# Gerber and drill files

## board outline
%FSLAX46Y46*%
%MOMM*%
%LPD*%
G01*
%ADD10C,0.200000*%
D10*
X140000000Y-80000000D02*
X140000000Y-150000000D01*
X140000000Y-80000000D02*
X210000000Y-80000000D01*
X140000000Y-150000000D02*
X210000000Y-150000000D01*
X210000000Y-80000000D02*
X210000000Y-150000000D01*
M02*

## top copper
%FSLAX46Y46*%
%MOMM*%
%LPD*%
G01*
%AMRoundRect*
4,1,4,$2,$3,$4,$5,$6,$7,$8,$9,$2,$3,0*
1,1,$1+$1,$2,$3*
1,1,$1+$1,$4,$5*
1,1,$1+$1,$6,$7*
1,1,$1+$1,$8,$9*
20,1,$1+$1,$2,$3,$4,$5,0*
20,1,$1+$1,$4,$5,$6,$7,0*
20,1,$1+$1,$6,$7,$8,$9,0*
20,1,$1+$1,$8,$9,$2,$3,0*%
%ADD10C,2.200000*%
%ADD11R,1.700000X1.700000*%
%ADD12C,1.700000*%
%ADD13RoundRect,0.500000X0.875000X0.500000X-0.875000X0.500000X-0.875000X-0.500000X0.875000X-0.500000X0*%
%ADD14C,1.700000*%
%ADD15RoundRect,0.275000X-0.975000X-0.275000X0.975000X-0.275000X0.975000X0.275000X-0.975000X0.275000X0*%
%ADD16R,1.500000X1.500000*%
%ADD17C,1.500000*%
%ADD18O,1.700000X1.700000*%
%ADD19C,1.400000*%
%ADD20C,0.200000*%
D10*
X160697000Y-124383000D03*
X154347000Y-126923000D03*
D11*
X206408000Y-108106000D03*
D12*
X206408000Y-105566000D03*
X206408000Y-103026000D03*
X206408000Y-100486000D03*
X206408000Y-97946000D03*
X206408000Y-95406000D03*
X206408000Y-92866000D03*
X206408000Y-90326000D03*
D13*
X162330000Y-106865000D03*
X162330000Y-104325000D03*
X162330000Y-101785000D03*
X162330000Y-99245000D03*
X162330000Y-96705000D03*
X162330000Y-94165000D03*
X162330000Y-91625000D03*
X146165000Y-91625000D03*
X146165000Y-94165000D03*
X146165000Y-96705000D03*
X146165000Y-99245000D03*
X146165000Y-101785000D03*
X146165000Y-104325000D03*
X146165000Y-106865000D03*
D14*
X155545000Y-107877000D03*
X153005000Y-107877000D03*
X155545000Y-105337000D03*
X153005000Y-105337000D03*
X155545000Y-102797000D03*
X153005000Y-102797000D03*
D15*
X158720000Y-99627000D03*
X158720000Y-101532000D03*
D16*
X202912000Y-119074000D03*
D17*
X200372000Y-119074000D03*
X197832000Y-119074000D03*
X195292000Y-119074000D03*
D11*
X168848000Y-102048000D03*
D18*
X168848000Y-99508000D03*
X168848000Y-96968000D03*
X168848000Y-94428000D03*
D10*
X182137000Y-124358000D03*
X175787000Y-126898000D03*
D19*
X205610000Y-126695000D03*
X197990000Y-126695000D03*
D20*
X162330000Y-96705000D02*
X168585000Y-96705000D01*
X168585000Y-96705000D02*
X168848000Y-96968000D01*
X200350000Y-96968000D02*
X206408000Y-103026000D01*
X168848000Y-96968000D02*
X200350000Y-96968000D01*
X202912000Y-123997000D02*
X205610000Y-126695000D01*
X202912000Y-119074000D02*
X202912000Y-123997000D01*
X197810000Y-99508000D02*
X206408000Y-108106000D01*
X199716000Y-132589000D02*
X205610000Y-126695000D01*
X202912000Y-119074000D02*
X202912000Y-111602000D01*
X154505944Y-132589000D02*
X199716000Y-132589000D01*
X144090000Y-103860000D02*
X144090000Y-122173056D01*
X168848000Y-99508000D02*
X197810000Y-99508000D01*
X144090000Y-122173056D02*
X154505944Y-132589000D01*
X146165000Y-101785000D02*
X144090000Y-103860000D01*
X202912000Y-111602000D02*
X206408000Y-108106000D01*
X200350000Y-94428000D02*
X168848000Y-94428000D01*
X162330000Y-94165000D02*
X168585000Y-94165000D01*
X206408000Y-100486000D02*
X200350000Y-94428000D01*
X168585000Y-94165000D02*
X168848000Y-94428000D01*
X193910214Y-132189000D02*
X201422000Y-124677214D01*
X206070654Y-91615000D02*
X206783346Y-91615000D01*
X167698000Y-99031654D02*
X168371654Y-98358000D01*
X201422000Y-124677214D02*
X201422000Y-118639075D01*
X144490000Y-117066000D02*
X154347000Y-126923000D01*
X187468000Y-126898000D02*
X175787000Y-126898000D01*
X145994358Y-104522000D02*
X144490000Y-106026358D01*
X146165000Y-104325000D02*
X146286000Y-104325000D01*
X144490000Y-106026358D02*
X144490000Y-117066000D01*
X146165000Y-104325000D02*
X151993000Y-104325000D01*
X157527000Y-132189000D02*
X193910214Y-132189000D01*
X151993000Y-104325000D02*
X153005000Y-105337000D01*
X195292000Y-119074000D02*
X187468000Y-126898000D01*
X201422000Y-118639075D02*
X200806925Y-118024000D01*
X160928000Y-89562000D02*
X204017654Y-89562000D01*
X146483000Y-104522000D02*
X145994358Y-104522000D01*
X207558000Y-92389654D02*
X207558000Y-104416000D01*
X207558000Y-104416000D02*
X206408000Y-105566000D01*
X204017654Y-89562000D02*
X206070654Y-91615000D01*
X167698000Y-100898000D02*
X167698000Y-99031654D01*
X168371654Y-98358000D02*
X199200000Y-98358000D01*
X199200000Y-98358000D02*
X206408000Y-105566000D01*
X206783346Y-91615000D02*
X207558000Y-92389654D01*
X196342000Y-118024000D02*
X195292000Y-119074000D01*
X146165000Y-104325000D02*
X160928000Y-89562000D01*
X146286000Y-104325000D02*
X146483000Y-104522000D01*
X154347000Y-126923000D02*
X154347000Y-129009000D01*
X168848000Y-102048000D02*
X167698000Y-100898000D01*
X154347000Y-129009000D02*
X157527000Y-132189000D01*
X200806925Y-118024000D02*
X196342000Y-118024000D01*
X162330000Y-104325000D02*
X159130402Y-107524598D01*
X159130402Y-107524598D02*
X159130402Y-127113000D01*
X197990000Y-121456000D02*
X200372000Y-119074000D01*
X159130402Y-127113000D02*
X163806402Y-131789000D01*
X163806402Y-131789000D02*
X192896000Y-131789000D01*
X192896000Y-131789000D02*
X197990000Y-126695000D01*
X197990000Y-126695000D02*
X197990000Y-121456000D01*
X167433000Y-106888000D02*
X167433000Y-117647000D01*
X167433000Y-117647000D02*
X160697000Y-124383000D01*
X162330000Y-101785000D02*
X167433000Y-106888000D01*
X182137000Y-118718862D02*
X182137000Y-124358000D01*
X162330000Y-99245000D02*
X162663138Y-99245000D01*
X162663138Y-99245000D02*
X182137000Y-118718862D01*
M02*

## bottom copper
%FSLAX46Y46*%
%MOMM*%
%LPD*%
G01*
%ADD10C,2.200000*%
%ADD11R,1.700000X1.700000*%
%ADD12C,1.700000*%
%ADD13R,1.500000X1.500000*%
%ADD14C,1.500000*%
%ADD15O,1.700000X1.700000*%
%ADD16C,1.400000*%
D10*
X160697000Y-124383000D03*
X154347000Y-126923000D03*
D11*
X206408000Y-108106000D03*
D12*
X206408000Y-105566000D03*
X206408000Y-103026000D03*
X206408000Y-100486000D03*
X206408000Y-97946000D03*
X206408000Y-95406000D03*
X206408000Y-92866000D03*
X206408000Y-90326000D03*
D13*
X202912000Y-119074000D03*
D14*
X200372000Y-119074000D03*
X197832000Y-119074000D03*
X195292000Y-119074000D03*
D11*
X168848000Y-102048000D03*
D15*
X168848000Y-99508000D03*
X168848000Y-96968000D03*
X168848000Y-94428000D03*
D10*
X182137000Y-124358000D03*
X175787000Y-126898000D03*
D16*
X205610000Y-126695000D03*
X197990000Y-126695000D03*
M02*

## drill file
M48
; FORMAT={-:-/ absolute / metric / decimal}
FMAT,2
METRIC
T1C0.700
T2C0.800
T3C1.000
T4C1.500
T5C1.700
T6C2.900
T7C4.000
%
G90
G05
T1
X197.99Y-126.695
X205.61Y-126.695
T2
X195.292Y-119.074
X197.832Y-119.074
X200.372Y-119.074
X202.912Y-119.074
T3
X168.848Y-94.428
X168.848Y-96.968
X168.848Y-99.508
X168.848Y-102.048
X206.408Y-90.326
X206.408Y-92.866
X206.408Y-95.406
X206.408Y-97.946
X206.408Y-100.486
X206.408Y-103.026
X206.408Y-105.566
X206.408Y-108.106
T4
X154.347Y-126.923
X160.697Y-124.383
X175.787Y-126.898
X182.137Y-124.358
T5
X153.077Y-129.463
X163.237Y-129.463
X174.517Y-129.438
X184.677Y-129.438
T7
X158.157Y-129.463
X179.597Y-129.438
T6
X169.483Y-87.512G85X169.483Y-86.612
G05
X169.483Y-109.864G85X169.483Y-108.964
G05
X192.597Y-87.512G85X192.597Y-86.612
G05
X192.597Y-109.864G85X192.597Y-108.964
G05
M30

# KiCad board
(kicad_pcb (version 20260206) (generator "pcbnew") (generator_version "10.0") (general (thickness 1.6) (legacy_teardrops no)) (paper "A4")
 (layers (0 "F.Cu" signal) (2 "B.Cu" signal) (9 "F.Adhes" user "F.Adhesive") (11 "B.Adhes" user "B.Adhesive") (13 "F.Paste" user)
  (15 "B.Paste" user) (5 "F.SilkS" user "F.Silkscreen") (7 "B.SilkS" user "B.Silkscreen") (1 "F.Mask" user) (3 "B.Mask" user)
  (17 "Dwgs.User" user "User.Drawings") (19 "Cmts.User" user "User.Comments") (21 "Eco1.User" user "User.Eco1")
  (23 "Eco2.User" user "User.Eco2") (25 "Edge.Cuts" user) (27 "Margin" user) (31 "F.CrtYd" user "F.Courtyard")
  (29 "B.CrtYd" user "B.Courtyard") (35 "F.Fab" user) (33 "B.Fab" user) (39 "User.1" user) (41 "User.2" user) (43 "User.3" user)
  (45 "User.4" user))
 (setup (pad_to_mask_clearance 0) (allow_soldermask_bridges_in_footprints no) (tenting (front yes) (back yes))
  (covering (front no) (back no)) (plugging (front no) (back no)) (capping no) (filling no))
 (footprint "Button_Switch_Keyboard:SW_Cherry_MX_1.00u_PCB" (layer "F.Cu") (at 160.697 124.383)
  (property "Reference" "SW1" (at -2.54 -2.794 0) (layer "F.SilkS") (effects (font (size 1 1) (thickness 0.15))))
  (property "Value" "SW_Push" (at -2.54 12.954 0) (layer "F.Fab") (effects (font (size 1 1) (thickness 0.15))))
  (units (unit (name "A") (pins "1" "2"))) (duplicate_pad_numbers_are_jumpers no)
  (pad "" np_thru_hole circle (at -7.62 5.08) (size 1.7 1.7) (drill 1.7) (layers "*.Cu" "*.Mask"))
  (pad "" np_thru_hole circle (at -2.54 5.08) (size 4 4) (drill 4) (layers "*.Cu" "*.Mask"))
  (pad "" np_thru_hole circle (at 2.54 5.08) (size 1.7 1.7) (drill 1.7) (layers "*.Cu" "*.Mask"))
  (pad "1" thru_hole circle (at 0 0) (size 2.2 2.2) (drill 1.5) (layers "*.Cu" "*.Mask") (remove_unused_layers no) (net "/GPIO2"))
  (pad "2" thru_hole circle (at -6.35 2.54) (size 2.2 2.2) (drill 1.5) (layers "*.Cu" "*.Mask") (remove_unused_layers no) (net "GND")))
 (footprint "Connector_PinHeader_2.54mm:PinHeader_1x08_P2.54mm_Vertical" (layer "F.Cu") (at 206.408 108.106 180)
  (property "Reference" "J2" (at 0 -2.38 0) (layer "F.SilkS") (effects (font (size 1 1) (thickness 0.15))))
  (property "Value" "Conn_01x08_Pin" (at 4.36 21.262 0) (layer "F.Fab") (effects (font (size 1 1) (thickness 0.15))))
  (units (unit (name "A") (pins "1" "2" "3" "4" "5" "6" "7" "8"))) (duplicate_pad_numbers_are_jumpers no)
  (pad "1" thru_hole rect (at 0 0 180) (size 1.7 1.7) (drill 1) (layers "*.Cu" "*.Mask") (remove_unused_layers no) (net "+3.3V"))
  (pad "2" thru_hole circle (at 0 2.54 180) (size 1.7 1.7) (drill 1) (layers "*.Cu" "*.Mask") (remove_unused_layers no) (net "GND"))
  (pad "3" thru_hole circle (at 0 5.08 180) (size 1.7 1.7) (drill 1) (layers "*.Cu" "*.Mask") (remove_unused_layers no) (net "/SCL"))
  (pad "4" thru_hole circle (at 0 7.62 180) (size 1.7 1.7) (drill 1) (layers "*.Cu" "*.Mask") (remove_unused_layers no) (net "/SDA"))
  (pad "5" thru_hole circle (at 0 10.16 180) (size 1.7 1.7) (drill 1) (layers "*.Cu" "*.Mask") (remove_unused_layers no)
   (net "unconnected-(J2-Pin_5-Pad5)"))
  (pad "6" thru_hole circle (at 0 12.7 180) (size 1.7 1.7) (drill 1) (layers "*.Cu" "*.Mask") (remove_unused_layers no)
   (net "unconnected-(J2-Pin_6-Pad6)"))
  (pad "7" thru_hole circle (at 0 15.24 180) (size 1.7 1.7) (drill 1) (layers "*.Cu" "*.Mask") (remove_unused_layers no)
   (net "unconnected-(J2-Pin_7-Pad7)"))
  (pad "8" thru_hole circle (at 0 17.78 180) (size 1.7 1.7) (drill 1) (layers "*.Cu" "*.Mask") (remove_unused_layers no)
   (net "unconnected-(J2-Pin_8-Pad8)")))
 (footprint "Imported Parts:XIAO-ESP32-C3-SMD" (layer "F.Cu") (at 163.165 88.745 180)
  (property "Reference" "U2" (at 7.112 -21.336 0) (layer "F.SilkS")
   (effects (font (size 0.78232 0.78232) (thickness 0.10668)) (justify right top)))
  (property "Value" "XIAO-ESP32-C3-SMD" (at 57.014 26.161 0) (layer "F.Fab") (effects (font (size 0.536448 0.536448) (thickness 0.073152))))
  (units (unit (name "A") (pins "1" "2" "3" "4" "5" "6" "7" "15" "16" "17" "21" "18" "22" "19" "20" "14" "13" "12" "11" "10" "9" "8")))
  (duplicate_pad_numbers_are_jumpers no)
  (pad "1" smd roundrect (at 0.835 -18.12 180) (size 2.75 2) (layers "F.Cu" "F.Mask" "F.Paste") (roundrect_rratio 0.25)
   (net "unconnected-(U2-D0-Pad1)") (solder_mask_margin 0.0508) (thermal_bridge_angle 45))
  (pad "2" smd roundrect (at 0.835 -15.58 180) (size 2.75 2) (layers "F.Cu" "F.Mask" "F.Paste") (roundrect_rratio 0.25) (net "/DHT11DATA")
   (solder_mask_margin 0.0508) (thermal_bridge_angle 45))
  (pad "3" smd roundrect (at 0.835 -13.04 180) (size 2.75 2) (layers "F.Cu" "F.Mask" "F.Paste") (roundrect_rratio 0.25) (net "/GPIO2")
   (solder_mask_margin 0.0508) (thermal_bridge_angle 45))
  (pad "4" smd roundrect (at 0.835 -10.5 180) (size 2.75 2) (layers "F.Cu" "F.Mask" "F.Paste") (roundrect_rratio 0.25) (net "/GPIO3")
   (solder_mask_margin 0.0508) (thermal_bridge_angle 45))
  (pad "5" smd roundrect (at 0.835 -7.96 180) (size 2.75 2) (layers "F.Cu" "F.Mask" "F.Paste") (roundrect_rratio 0.25) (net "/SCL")
   (solder_mask_margin 0.0508) (thermal_bridge_angle 45))
  (pad "6" smd roundrect (at 0.835 -5.42 180) (size 2.75 2) (layers "F.Cu" "F.Mask" "F.Paste") (roundrect_rratio 0.25) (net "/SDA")
   (solder_mask_margin 0.0508) (thermal_bridge_angle 45))
  (pad "7" smd roundrect (at 0.835 -2.88 180) (size 2.75 2) (layers "F.Cu" "F.Mask" "F.Paste") (roundrect_rratio 0.25)
   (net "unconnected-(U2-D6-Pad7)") (solder_mask_margin 0.0508) (thermal_bridge_angle 45))
  (pad "8" smd roundrect (at 17 -2.88 180) (size 2.75 2) (layers "F.Cu" "F.Mask" "F.Paste") (roundrect_rratio 0.25)
   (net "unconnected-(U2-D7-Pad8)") (solder_mask_margin 0.0508) (thermal_bridge_angle 45))
  (pad "9" smd roundrect (at 17 -5.42 180) (size 2.75 2) (layers "F.Cu" "F.Mask" "F.Paste") (roundrect_rratio 0.25)
   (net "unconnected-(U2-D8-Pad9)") (solder_mask_margin 0.0508) (thermal_bridge_angle 45))
  (pad "10" smd roundrect (at 17 -7.96 180) (size 2.75 2) (layers "F.Cu" "F.Mask" "F.Paste") (roundrect_rratio 0.25)
   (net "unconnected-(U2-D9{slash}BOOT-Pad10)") (solder_mask_margin 0.0508) (thermal_bridge_angle 45))
  (pad "11" smd roundrect (at 17 -10.5 180) (size 2.75 2) (layers "F.Cu" "F.Mask" "F.Paste") (roundrect_rratio 0.25)
   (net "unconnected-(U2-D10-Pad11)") (solder_mask_margin 0.0508) (thermal_bridge_angle 45))
  (pad "12" smd roundrect (at 17 -13.04 180) (size 2.75 2) (layers "F.Cu" "F.Mask" "F.Paste") (roundrect_rratio 0.25) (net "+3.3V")
   (solder_mask_margin 0.0508) (thermal_bridge_angle 45))
  (pad "13" smd roundrect (at 17 -15.58 180) (size 2.75 2) (layers "F.Cu" "F.Mask" "F.Paste") (roundrect_rratio 0.25) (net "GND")
   (solder_mask_margin 0.0508) (thermal_bridge_angle 45))
  (pad "14" smd roundrect (at 17 -18.12 180) (size 2.75 2) (layers "F.Cu" "F.Mask" "F.Paste") (roundrect_rratio 0.25) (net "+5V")
   (solder_mask_margin 0.0508) (thermal_bridge_angle 45))
  (pad "15" smd circle (at 7.62 -19.132 180) (size 1.7 1.7) (layers "F.Cu" "F.Mask" "F.Paste") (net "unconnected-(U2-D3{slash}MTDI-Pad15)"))
  (pad "16" smd circle (at 10.16 -19.132 180) (size 1.7 1.7) (layers "F.Cu" "F.Mask" "F.Paste") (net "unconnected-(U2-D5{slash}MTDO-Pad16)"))
  (pad "17" smd circle (at 7.62 -16.592 180) (size 1.7 1.7) (layers "F.Cu" "F.Mask" "F.Paste") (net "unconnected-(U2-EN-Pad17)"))
  (pad "18" smd circle (at 10.16 -16.592 180) (size 1.7 1.7) (layers "F.Cu" "F.Mask" "F.Paste") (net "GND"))
  (pad "19" smd circle (at 7.62 -14.052 180) (size 1.7 1.7) (layers "F.Cu" "F.Mask" "F.Paste") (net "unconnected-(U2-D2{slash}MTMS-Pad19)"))
  (pad "20" smd circle (at 10.16 -14.052 180) (size 1.7 1.7) (layers "F.Cu" "F.Mask" "F.Paste") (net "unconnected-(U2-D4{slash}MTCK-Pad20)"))
  (pad "21" smd roundrect (at 4.445 -10.882) (size 2.5 1.1) (layers "F.Cu" "F.Mask" "F.Paste") (roundrect_rratio 0.25)
   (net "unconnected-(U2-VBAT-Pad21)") (thermal_bridge_angle 45))
  (pad "22" smd roundrect (at 4.445 -12.787) (size 2.5 1.1) (layers "F.Cu" "F.Mask" "F.Paste") (roundrect_rratio 0.25)
   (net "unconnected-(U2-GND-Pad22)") (thermal_bridge_angle 45)))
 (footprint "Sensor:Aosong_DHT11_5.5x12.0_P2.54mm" (layer "F.Cu") (at 202.912 119.074 -90)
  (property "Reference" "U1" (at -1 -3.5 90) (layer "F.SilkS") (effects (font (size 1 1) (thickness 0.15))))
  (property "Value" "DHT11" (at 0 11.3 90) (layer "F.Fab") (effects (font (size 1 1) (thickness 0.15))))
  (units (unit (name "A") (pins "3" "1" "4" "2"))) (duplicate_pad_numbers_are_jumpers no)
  (pad "1" thru_hole rect (at 0 0 270) (size 1.5 1.5) (drill 0.8) (layers "*.Cu" "*.Mask") (remove_unused_layers no) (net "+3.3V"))
  (pad "2" thru_hole circle (at 0 2.54 270) (size 1.5 1.5) (drill 0.8) (layers "*.Cu" "*.Mask") (remove_unused_layers no) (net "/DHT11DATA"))
  (pad "3" thru_hole circle (at 0 5.08 270) (size 1.5 1.5) (drill 0.8) (layers "*.Cu" "*.Mask") (remove_unused_layers no)
   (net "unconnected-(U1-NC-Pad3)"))
  (pad "4" thru_hole circle (at 0 7.62 270) (size 1.5 1.5) (drill 0.8) (layers "*.Cu" "*.Mask") (remove_unused_layers no) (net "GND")))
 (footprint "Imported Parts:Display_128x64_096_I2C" (layer "F.Cu") (at 168.848 98.238 90)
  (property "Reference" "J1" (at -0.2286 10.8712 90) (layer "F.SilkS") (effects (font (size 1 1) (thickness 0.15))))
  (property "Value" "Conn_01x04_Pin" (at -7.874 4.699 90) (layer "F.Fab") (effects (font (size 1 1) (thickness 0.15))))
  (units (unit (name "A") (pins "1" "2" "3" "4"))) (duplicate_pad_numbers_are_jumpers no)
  (pad "" np_thru_hole oval (at -11.176 0.635 90) (size 3.8 2.9) (drill oval 3.8 2.9) (layers "*.Cu" "*.Mask"))
  (pad "" np_thru_hole oval (at -11.176 23.749 90) (size 3.8 2.9) (drill oval 3.8 2.9) (layers "*.Cu" "*.Mask"))
  (pad "" np_thru_hole oval (at 11.176 0.635 90) (size 3.8 2.9) (drill oval 3.8 2.9) (layers "*.Cu" "*.Mask"))
  (pad "" np_thru_hole oval (at 11.176 23.749 90) (size 3.8 2.9) (drill oval 3.8 2.9) (layers "*.Cu" "*.Mask"))
  (pad "1" thru_hole rect (at -3.81 0 180) (size 1.7 1.7) (drill 1) (layers "*.Cu" "*.Mask") (remove_unused_layers no) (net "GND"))
  (pad "2" thru_hole oval (at -1.27 0 180) (size 1.7 1.7) (drill 1) (layers "*.Cu" "*.Mask") (remove_unused_layers no) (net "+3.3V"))
  (pad "3" thru_hole oval (at 1.27 0 180) (size 1.7 1.7) (drill 1) (layers "*.Cu" "*.Mask") (remove_unused_layers no) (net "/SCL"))
  (pad "4" thru_hole oval (at 3.81 0 180) (size 1.7 1.7) (drill 1) (layers "*.Cu" "*.Mask") (remove_unused_layers no) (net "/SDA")))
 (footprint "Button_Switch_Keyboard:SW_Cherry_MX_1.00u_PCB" (layer "F.Cu") (at 182.137 124.358)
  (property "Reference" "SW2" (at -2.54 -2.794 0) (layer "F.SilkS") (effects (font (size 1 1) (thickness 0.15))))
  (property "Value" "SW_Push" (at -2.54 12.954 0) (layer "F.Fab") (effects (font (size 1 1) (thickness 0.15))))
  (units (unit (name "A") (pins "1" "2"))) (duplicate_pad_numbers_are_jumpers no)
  (pad "" np_thru_hole circle (at -7.62 5.08) (size 1.7 1.7) (drill 1.7) (layers "*.Cu" "*.Mask"))
  (pad "" np_thru_hole circle (at -2.54 5.08) (size 4 4) (drill 4) (layers "*.Cu" "*.Mask"))
  (pad "" np_thru_hole circle (at 2.54 5.08) (size 1.7 1.7) (drill 1.7) (layers "*.Cu" "*.Mask"))
  (pad "1" thru_hole circle (at 0 0) (size 2.2 2.2) (drill 1.5) (layers "*.Cu" "*.Mask") (remove_unused_layers no) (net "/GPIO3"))
  (pad "2" thru_hole circle (at -6.35 2.54) (size 2.2 2.2) (drill 1.5) (layers "*.Cu" "*.Mask") (remove_unused_layers no) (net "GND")))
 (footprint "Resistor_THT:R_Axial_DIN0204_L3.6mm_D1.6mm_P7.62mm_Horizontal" (layer "F.Cu") (at 205.61 126.695 180)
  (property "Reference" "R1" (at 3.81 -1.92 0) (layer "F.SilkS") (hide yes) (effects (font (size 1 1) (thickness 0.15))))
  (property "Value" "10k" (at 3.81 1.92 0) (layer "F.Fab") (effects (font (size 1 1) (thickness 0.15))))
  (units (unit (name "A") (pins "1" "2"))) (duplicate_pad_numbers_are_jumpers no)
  (pad "1" thru_hole circle (at 0 0 180) (size 1.4 1.4) (drill 0.7) (layers "*.Cu" "*.Mask") (remove_unused_layers no) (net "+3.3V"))
  (pad "2" thru_hole circle (at 7.62 0 180) (size 1.4 1.4) (drill 0.7) (layers "*.Cu" "*.Mask") (remove_unused_layers no) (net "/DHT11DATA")))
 (gr_line (start 140 80) (end 140 150) (stroke (width 0.2) (type default)) (layer "Edge.Cuts"))
 (gr_line (start 140 80) (end 210 80) (stroke (width 0.2) (type default)) (layer "Edge.Cuts"))
 (gr_line (start 140 150) (end 210 150) (stroke (width 0.2) (type default)) (layer "Edge.Cuts"))
 (gr_line (start 210 80) (end 210 150) (stroke (width 0.2) (type default)) (layer "Edge.Cuts"))
 (segment (start 162.33 96.705) (end 168.585 96.705) (width 0.2) (layer "F.Cu") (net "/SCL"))
 (segment (start 168.585 96.705) (end 168.848 96.968) (width 0.2) (layer "F.Cu") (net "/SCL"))
 (segment (start 200.35 96.968) (end 206.408 103.026) (width 0.2) (layer "F.Cu") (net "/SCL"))
 (segment (start 168.848 96.968) (end 200.35 96.968) (width 0.2) (layer "F.Cu") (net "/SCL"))
 (segment (start 202.912 123.997) (end 205.61 126.695) (width 0.2) (layer "F.Cu") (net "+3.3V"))
 (segment (start 202.912 119.074) (end 202.912 123.997) (width 0.2) (layer "F.Cu") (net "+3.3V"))
 (segment (start 197.81 99.508) (end 206.408 108.106) (width 0.2) (layer "F.Cu") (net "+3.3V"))
 (segment (start 199.716 132.589) (end 205.61 126.695) (width 0.2) (layer "F.Cu") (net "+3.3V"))
 (segment (start 202.912 119.074) (end 202.912 111.602) (width 0.2) (layer "F.Cu") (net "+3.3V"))
 (segment (start 154.505944 132.589) (end 199.716 132.589) (width 0.2) (layer "F.Cu") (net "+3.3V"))
 (segment (start 144.09 103.86) (end 144.09 122.173056) (width 0.2) (layer "F.Cu") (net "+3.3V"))
 (segment (start 168.848 99.508) (end 197.81 99.508) (width 0.2) (layer "F.Cu") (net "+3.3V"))
 (segment (start 144.09 122.173056) (end 154.505944 132.589) (width 0.2) (layer "F.Cu") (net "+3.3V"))
 (segment (start 146.165 101.785) (end 144.09 103.86) (width 0.2) (layer "F.Cu") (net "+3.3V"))
 (segment (start 202.912 111.602) (end 206.408 108.106) (width 0.2) (layer "F.Cu") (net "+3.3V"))
 (segment (start 200.35 94.428) (end 168.848 94.428) (width 0.2) (layer "F.Cu") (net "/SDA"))
 (segment (start 162.33 94.165) (end 168.585 94.165) (width 0.2) (layer "F.Cu") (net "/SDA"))
 (segment (start 206.408 100.486) (end 200.35 94.428) (width 0.2) (layer "F.Cu") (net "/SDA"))
 (segment (start 168.585 94.165) (end 168.848 94.428) (width 0.2) (layer "F.Cu") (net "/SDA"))
 (segment (start 193.910214 132.189) (end 201.422 124.677214) (width 0.2) (layer "F.Cu") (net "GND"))
 (segment (start 206.070654 91.615) (end 206.783346 91.615) (width 0.2) (layer "F.Cu") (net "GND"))
 (segment (start 167.698 99.031654) (end 168.371654 98.358) (width 0.2) (layer "F.Cu") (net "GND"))
 (segment (start 201.422 124.677214) (end 201.422 118.639075) (width 0.2) (layer "F.Cu") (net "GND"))
 (segment (start 144.49 117.066) (end 154.347 126.923) (width 0.2) (layer "F.Cu") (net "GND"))
 (segment (start 187.468 126.898) (end 175.787 126.898) (width 0.2) (layer "F.Cu") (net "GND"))
 (segment (start 145.994358 104.522) (end 144.49 106.026358) (width 0.2) (layer "F.Cu") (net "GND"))
 (segment (start 146.165 104.325) (end 146.286 104.325) (width 0.2) (layer "F.Cu") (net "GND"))
 (segment (start 144.49 106.026358) (end 144.49 117.066) (width 0.2) (layer "F.Cu") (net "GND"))
 (segment (start 146.165 104.325) (end 151.993 104.325) (width 0.2) (layer "F.Cu") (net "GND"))
 (segment (start 157.527 132.189) (end 193.910214 132.189) (width 0.2) (layer "F.Cu") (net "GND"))
 (segment (start 151.993 104.325) (end 153.005 105.337) (width 0.2) (layer "F.Cu") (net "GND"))
 (segment (start 195.292 119.074) (end 187.468 126.898) (width 0.2) (layer "F.Cu") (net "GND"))
 (segment (start 201.422 118.639075) (end 200.806925 118.024) (width 0.2) (layer "F.Cu") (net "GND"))
 (segment (start 160.928 89.562) (end 204.017654 89.562) (width 0.2) (layer "F.Cu") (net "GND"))
 (segment (start 146.483 104.522) (end 145.994358 104.522) (width 0.2) (layer "F.Cu") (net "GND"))
 (segment (start 207.558 92.389654) (end 207.558 104.416) (width 0.2) (layer "F.Cu") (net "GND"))
 (segment (start 207.558 104.416) (end 206.408 105.566) (width 0.2) (layer "F.Cu") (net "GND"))
 (segment (start 204.017654 89.562) (end 206.070654 91.615) (width 0.2) (layer "F.Cu") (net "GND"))
 (segment (start 167.698 100.898) (end 167.698 99.031654) (width 0.2) (layer "F.Cu") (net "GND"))
 (segment (start 168.371654 98.358) (end 199.2 98.358) (width 0.2) (layer "F.Cu") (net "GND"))
 (segment (start 199.2 98.358) (end 206.408 105.566) (width 0.2) (layer "F.Cu") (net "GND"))
 (segment (start 206.783346 91.615) (end 207.558 92.389654) (width 0.2) (layer "F.Cu") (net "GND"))
 (segment (start 196.342 118.024) (end 195.292 119.074) (width 0.2) (layer "F.Cu") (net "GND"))
 (segment (start 146.165 104.325) (end 160.928 89.562) (width 0.2) (layer "F.Cu") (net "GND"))
 (segment (start 146.286 104.325) (end 146.483 104.522) (width 0.2) (layer "F.Cu") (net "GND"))
 (segment (start 154.347 126.923) (end 154.347 129.009) (width 0.2) (layer "F.Cu") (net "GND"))
 (segment (start 168.848 102.048) (end 167.698 100.898) (width 0.2) (layer "F.Cu") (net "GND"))
 (segment (start 154.347 129.009) (end 157.527 132.189) (width 0.2) (layer "F.Cu") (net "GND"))
 (segment (start 200.806925 118.024) (end 196.342 118.024) (width 0.2) (layer "F.Cu") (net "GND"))
 (segment (start 162.33 104.325) (end 159.130402 107.524598) (width 0.2) (layer "F.Cu") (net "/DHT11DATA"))
 (segment (start 159.130402 107.524598) (end 159.130402 127.113) (width 0.2) (layer "F.Cu") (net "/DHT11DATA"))
 (segment (start 197.99 121.456) (end 200.372 119.074) (width 0.2) (layer "F.Cu") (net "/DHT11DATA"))
 (segment (start 159.130402 127.113) (end 163.806402 131.789) (width 0.2) (layer "F.Cu") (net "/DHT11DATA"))
 (segment (start 163.806402 131.789) (end 192.896 131.789) (width 0.2) (layer "F.Cu") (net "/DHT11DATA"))
 (segment (start 192.896 131.789) (end 197.99 126.695) (width 0.2) (layer "F.Cu") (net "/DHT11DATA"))
 (segment (start 197.99 126.695) (end 197.99 121.456) (width 0.2) (layer "F.Cu") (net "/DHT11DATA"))
 (segment (start 167.433 106.888) (end 167.433 117.647) (width 0.2) (layer "F.Cu") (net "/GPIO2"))
 (segment (start 167.433 117.647) (end 160.697 124.383) (width 0.2) (layer "F.Cu") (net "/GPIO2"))
 (segment (start 162.33 101.785) (end 167.433 106.888) (width 0.2) (layer "F.Cu") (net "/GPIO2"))
 (segment (start 182.137 118.718862) (end 182.137 124.358) (width 0.2) (layer "F.Cu") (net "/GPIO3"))
 (segment (start 162.33 99.245) (end 162.663138 99.245) (width 0.2) (layer "F.Cu") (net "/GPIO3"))
 (segment (start 162.663138 99.245) (end 182.137 118.718862) (width 0.2) (layer "F.Cu") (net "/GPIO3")))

